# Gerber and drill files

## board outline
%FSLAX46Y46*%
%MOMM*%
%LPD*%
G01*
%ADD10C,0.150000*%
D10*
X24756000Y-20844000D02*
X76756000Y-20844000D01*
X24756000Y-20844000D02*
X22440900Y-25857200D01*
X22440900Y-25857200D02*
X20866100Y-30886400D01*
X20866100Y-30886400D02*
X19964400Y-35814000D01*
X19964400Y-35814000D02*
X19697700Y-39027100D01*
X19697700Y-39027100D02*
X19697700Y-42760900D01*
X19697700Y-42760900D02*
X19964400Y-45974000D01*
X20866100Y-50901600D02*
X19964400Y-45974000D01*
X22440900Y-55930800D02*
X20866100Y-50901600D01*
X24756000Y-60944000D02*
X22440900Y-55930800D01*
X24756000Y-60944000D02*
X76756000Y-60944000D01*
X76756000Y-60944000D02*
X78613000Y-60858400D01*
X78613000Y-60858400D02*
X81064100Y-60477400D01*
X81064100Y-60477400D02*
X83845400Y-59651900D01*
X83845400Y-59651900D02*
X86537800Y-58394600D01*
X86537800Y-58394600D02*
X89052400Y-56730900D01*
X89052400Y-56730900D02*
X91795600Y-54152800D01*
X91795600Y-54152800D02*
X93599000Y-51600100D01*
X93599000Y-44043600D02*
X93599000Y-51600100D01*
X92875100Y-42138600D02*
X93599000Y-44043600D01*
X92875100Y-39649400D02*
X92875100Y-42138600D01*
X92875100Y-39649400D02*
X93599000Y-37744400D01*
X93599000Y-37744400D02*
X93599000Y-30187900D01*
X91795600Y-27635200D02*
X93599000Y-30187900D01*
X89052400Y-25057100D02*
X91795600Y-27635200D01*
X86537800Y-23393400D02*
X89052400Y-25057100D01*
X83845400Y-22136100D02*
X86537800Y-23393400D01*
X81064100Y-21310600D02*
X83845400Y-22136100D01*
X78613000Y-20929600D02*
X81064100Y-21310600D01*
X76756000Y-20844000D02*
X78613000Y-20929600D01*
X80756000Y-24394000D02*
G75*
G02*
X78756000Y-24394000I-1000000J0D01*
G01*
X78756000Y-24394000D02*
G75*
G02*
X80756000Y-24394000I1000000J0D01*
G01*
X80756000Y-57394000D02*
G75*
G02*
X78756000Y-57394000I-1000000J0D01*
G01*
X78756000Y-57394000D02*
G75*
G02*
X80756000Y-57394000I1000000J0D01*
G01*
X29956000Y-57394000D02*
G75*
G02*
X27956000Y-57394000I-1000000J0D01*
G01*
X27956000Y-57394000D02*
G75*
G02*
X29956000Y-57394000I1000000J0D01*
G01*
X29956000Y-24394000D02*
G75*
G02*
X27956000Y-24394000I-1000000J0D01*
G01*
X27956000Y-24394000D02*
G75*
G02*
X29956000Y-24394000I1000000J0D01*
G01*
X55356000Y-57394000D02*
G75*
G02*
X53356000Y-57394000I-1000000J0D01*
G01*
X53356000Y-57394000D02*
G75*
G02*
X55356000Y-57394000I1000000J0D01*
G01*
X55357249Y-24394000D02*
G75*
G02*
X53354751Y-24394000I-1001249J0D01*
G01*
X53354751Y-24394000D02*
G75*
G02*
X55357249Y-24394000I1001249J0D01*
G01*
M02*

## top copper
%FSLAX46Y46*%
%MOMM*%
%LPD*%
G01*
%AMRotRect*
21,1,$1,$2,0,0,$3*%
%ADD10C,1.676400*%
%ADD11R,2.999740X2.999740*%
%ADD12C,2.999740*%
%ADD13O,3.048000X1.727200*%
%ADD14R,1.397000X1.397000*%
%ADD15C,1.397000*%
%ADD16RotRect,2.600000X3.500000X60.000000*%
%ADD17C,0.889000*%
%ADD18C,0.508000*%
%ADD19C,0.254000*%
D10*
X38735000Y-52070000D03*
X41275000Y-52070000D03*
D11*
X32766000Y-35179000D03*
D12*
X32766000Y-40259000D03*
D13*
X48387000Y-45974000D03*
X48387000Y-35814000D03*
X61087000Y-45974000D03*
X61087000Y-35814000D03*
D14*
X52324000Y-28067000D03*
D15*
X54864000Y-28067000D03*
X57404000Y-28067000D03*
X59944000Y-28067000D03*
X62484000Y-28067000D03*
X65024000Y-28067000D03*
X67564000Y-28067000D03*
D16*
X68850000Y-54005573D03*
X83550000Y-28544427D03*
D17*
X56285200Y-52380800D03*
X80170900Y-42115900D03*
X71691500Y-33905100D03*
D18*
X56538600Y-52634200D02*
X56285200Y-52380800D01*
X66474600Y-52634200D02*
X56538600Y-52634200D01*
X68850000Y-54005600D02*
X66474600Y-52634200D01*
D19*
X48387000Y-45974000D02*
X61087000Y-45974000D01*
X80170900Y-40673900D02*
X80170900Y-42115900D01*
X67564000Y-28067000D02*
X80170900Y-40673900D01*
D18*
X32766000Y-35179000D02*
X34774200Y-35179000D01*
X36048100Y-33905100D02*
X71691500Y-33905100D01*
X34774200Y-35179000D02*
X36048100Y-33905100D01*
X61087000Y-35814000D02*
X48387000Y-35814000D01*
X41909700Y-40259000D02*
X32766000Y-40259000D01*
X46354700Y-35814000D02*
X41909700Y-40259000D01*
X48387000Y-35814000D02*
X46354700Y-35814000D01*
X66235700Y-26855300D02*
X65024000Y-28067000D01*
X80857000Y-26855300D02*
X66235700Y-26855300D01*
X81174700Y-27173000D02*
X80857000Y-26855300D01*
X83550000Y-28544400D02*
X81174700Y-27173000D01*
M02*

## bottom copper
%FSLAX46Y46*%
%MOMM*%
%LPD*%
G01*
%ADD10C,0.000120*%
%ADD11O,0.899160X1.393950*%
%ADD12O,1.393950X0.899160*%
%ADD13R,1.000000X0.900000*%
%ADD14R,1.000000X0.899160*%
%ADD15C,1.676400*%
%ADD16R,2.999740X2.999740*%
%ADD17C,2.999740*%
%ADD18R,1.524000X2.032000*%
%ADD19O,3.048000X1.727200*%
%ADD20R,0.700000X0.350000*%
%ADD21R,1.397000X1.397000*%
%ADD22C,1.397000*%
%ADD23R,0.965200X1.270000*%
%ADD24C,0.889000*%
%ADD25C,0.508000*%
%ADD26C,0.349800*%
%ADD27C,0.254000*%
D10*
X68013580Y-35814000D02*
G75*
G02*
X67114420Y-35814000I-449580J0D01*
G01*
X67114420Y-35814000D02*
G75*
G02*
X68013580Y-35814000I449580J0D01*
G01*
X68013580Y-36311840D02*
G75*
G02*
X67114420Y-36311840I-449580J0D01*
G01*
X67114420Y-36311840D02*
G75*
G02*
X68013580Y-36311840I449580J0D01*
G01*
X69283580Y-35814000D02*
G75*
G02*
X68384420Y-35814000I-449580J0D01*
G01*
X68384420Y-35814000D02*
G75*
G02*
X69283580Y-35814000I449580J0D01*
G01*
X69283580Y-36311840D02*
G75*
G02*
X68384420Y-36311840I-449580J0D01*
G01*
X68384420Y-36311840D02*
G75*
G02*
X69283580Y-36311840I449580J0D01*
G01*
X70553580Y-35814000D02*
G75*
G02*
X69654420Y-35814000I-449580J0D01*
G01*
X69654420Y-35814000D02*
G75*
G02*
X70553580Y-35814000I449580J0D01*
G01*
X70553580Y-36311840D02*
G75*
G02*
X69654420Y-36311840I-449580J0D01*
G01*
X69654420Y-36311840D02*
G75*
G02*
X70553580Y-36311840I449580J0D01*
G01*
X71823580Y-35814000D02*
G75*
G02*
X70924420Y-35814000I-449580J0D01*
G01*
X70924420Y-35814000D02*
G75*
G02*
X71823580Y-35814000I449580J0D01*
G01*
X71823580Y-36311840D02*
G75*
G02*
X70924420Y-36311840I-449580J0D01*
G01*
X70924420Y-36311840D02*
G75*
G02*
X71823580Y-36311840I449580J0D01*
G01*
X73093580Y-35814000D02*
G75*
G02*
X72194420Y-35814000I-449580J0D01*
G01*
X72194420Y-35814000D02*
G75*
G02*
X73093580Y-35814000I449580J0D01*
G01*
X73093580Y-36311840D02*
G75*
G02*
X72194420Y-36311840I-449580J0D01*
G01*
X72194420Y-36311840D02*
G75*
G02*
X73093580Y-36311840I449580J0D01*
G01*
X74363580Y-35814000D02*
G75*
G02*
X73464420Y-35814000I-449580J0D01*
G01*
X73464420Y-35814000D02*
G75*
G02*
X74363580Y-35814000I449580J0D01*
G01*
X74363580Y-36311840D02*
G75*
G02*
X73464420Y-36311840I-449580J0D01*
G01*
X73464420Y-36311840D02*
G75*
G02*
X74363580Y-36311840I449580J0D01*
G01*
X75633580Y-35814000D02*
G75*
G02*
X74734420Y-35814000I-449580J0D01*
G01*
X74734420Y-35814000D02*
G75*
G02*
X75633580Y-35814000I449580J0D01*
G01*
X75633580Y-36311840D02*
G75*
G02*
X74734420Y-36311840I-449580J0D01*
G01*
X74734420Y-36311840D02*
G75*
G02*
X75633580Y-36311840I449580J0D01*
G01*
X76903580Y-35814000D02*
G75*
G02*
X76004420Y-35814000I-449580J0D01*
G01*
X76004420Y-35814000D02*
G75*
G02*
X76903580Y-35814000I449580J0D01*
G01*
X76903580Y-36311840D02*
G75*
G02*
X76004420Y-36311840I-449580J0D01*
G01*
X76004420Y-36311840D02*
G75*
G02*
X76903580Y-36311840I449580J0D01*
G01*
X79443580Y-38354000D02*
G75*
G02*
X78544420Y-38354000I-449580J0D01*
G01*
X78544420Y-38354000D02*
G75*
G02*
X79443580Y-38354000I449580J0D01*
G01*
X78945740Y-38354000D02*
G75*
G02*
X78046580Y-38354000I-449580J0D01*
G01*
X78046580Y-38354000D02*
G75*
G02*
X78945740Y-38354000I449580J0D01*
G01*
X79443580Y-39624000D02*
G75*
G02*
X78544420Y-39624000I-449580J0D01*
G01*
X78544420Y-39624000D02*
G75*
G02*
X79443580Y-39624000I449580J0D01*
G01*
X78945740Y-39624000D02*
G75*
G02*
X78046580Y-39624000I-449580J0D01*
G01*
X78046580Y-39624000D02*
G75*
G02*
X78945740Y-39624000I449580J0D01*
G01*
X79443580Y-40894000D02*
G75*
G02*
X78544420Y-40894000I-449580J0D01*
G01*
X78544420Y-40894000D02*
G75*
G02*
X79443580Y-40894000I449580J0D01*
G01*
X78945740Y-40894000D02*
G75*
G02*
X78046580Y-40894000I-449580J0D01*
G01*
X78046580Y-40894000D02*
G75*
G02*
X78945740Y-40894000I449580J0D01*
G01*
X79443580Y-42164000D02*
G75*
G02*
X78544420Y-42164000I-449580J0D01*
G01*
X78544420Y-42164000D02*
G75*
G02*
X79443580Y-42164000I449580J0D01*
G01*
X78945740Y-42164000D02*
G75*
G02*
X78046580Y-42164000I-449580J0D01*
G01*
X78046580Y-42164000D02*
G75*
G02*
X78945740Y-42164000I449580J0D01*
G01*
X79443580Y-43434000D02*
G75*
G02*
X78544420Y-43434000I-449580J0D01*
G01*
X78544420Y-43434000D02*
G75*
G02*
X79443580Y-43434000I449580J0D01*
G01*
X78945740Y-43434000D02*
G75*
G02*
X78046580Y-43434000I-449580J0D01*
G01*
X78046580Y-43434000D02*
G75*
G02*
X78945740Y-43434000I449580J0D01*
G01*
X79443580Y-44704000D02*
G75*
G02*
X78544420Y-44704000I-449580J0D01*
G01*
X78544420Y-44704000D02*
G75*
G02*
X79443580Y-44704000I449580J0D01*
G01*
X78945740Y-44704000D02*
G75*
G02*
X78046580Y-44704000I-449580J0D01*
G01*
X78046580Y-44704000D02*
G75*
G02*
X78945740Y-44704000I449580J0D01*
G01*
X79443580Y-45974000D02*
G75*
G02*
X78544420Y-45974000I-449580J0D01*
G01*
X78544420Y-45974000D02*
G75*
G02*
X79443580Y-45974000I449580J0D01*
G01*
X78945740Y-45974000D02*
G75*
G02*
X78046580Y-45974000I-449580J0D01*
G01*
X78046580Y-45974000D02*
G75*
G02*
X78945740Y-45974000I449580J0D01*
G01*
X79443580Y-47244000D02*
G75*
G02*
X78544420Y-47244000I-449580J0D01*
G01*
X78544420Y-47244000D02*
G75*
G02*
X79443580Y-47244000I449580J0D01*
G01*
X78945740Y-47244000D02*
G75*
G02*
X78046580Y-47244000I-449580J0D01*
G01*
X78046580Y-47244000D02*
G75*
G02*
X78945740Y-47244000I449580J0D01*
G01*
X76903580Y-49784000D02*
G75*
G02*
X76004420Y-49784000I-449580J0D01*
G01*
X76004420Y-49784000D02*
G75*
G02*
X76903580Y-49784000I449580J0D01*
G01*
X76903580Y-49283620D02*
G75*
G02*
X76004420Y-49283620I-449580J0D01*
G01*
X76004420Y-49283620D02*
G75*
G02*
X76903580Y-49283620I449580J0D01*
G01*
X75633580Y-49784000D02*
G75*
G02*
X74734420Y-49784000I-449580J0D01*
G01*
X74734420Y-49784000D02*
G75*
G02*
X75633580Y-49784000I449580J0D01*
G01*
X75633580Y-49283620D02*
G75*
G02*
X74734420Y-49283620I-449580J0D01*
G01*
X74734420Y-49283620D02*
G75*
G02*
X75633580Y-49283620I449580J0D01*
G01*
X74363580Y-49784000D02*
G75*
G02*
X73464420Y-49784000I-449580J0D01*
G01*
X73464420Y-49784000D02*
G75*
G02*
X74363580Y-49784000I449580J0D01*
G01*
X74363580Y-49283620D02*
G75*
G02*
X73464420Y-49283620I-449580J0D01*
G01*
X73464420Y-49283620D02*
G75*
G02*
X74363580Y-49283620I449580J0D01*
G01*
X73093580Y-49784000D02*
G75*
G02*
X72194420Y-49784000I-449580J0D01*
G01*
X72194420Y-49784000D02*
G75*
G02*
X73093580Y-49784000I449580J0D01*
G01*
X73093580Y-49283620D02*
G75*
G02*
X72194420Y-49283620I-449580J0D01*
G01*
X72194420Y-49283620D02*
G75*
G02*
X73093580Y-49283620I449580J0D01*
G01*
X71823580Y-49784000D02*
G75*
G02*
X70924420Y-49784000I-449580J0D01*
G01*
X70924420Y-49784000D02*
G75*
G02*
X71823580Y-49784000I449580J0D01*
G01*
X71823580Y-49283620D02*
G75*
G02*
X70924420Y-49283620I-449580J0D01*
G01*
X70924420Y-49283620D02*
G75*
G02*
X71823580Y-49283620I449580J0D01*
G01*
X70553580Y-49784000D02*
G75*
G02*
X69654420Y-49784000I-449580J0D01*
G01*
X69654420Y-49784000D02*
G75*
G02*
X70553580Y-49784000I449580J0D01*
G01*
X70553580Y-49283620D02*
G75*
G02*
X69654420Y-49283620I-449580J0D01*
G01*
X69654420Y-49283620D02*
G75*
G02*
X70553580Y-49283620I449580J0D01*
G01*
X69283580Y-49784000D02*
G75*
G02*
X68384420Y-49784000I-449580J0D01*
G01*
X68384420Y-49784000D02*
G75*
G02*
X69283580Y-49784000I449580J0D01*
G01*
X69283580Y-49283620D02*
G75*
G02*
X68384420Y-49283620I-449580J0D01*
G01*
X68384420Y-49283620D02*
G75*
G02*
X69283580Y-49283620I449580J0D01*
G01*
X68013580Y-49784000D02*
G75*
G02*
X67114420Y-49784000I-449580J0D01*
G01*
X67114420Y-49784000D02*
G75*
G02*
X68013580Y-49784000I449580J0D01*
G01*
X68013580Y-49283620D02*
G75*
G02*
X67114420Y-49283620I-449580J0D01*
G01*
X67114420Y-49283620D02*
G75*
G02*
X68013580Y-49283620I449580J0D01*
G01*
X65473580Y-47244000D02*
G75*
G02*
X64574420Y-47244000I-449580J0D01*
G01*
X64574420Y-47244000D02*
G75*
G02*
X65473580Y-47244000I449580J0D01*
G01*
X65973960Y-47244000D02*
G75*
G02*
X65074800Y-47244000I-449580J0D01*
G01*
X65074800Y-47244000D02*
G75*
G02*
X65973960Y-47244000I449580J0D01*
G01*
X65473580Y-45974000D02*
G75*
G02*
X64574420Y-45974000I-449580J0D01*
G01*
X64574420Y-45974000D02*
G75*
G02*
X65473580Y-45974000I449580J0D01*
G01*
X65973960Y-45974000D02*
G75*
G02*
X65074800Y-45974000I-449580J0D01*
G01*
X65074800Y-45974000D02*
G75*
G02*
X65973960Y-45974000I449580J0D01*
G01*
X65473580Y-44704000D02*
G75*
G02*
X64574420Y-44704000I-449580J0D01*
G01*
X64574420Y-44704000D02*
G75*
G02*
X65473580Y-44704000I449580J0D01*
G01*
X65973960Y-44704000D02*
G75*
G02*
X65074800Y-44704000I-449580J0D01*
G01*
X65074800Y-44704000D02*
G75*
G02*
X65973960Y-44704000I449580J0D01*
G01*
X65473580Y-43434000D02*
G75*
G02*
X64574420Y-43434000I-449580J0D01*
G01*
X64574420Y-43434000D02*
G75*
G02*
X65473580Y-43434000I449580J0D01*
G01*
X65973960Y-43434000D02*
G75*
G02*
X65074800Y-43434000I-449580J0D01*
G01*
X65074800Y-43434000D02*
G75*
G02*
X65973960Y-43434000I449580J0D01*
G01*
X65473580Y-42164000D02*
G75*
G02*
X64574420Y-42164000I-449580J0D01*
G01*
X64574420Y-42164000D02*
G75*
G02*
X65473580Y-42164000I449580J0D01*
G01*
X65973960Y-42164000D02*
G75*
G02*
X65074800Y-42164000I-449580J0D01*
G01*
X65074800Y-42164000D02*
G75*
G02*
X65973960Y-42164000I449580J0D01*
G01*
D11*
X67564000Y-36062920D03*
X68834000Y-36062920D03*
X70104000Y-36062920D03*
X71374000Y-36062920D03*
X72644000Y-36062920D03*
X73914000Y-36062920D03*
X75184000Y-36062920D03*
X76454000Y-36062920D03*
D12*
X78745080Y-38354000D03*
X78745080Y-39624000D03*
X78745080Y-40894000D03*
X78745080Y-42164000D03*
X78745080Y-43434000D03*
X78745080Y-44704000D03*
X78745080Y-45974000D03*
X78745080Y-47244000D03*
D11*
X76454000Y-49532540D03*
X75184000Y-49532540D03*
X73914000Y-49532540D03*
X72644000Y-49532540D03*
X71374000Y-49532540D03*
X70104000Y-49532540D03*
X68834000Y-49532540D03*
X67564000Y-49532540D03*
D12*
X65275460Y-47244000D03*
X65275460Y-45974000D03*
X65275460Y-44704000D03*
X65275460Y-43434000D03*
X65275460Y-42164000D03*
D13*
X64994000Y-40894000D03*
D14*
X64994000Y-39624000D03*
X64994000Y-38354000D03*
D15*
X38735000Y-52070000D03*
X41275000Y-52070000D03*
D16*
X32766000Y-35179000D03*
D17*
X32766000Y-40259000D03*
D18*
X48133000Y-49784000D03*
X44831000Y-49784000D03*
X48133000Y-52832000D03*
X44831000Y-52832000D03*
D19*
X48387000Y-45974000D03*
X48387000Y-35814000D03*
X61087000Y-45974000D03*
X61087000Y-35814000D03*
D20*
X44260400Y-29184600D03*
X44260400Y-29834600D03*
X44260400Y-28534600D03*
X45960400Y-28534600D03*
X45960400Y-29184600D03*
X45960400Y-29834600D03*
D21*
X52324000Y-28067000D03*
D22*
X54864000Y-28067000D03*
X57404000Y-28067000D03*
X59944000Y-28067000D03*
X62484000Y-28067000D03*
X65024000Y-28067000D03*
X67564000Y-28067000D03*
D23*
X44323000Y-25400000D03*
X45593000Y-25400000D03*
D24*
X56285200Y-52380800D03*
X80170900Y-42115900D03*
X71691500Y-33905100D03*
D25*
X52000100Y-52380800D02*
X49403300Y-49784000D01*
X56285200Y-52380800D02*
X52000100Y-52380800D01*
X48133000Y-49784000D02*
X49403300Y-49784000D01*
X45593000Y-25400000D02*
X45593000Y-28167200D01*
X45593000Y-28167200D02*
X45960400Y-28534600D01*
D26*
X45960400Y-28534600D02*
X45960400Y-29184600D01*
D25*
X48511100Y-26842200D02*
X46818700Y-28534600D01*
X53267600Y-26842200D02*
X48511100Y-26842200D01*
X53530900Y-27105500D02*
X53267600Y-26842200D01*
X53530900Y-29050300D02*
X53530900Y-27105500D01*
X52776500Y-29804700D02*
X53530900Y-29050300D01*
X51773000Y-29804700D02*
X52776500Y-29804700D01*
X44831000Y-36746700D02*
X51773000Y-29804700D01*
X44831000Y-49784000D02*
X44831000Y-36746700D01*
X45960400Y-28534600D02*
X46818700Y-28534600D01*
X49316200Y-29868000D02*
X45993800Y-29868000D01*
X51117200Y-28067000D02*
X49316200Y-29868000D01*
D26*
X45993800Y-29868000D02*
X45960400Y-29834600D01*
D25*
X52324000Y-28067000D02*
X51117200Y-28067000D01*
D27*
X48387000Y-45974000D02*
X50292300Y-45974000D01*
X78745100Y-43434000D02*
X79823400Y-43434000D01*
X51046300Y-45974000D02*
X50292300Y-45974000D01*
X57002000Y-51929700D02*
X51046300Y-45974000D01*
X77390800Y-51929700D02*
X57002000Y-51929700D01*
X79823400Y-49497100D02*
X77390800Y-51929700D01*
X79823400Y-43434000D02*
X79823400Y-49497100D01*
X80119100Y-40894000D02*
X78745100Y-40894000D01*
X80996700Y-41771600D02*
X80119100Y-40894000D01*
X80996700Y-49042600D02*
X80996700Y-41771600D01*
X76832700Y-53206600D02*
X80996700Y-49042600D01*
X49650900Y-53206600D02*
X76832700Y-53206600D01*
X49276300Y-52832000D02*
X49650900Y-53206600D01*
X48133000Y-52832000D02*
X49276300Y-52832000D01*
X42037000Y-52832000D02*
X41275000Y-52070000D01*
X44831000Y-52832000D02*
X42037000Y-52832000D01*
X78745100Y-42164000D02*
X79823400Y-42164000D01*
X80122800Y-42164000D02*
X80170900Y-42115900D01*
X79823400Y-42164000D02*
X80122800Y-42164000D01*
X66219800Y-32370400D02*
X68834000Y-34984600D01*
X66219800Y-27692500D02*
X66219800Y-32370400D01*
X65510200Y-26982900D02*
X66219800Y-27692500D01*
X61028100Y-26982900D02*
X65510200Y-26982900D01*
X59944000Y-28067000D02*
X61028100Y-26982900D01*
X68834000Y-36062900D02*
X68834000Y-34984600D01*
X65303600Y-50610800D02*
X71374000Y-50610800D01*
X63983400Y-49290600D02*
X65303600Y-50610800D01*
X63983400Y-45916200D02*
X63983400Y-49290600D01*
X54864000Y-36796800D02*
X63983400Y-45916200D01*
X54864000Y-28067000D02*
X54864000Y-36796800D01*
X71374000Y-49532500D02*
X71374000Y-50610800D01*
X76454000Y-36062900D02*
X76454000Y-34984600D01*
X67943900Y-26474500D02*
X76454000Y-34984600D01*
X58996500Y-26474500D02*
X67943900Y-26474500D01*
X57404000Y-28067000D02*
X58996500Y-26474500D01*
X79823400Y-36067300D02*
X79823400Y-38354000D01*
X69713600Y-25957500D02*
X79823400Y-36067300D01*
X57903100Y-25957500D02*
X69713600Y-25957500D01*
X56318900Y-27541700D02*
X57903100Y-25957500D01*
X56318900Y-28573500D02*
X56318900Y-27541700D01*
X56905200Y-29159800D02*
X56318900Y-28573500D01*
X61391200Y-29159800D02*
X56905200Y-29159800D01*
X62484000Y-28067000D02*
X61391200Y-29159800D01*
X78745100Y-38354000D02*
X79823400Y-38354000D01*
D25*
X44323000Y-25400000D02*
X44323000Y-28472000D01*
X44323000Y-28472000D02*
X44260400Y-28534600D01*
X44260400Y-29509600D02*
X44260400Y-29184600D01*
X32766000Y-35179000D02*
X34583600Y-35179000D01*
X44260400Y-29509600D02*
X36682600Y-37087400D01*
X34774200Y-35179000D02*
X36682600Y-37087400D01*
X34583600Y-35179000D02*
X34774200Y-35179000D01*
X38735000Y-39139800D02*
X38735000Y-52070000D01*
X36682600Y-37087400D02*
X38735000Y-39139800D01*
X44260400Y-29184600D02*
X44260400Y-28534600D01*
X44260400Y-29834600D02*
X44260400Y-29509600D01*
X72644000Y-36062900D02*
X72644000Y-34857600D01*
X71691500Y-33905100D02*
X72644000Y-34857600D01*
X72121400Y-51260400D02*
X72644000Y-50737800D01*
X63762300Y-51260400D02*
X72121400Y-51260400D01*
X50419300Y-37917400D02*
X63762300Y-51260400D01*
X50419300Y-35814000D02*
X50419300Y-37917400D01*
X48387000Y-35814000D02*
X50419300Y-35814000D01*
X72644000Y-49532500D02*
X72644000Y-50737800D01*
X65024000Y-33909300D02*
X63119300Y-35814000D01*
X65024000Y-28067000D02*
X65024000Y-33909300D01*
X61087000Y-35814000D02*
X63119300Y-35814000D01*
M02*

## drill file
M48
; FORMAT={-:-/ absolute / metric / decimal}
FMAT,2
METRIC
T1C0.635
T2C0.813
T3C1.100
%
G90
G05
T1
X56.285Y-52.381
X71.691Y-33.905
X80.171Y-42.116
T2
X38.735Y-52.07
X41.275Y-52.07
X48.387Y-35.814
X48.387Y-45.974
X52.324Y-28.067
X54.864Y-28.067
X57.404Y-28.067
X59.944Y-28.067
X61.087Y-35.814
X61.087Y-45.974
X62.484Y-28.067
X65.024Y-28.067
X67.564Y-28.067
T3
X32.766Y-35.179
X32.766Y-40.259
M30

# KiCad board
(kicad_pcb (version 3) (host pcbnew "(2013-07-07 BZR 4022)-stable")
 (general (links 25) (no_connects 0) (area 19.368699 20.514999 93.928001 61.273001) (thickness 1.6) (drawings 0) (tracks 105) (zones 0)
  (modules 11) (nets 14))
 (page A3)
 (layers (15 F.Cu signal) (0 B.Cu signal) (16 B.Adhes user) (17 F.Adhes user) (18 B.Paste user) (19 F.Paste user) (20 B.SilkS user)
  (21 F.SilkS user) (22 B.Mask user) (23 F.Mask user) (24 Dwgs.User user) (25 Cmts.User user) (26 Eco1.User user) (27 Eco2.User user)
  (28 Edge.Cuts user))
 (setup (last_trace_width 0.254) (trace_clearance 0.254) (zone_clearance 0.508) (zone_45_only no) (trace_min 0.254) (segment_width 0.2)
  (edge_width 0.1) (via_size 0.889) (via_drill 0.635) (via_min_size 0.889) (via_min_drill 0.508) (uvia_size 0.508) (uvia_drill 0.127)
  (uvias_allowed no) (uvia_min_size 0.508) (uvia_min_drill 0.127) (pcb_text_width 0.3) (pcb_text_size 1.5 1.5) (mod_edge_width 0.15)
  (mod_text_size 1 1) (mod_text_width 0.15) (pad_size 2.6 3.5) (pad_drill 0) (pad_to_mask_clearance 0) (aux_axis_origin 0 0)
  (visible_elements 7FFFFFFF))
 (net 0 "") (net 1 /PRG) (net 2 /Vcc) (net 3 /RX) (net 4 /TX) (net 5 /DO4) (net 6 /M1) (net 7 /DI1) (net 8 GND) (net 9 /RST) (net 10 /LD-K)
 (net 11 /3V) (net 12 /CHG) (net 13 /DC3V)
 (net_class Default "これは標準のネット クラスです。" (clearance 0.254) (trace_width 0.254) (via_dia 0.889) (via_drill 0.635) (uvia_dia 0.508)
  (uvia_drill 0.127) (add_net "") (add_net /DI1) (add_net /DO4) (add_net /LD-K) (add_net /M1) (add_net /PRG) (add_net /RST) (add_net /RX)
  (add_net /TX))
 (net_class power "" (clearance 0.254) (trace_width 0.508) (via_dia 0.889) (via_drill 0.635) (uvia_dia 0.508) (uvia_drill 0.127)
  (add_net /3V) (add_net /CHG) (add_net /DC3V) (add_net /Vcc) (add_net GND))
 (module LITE (layer B.Cu) (at 78.994 35.814 270)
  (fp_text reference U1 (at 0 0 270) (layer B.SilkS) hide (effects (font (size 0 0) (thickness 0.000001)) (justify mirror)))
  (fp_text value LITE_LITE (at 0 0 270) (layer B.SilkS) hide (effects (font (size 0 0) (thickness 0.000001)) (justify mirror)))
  (fp_circle (center 0 11.43) (end 0.44958 11.43) (layer B.Cu) (width 0.00012))
  (fp_circle (center 0.49784 11.43) (end 0.94742 11.43) (layer B.Cu) (width 0.00012))
  (fp_circle (center 0 10.16) (end 0.44958 10.16) (layer B.Cu) (width 0.00012))
  (fp_circle (center 0.49784 10.16) (end 0.94742 10.16) (layer B.Cu) (width 0.00012))
  (fp_circle (center 0 8.89) (end 0.44958 8.89) (layer B.Cu) (width 0.00012))
  (fp_circle (center 0.49784 8.89) (end 0.94742 8.89) (layer B.Cu) (width 0.00012))
  (fp_circle (center 0 7.62) (end 0.44958 7.62) (layer B.Cu) (width 0.00012))
  (fp_circle (center 0.49784 7.62) (end 0.94742 7.62) (layer B.Cu) (width 0.00012))
  (fp_circle (center 0 6.35) (end 0.44958 6.35) (layer B.Cu) (width 0.00012))
  (fp_circle (center 0.49784 6.35) (end 0.94742 6.35) (layer B.Cu) (width 0.00012))
  (fp_circle (center 0 5.08) (end 0.44958 5.08) (layer B.Cu) (width 0.00012))
  (fp_circle (center 0.49784 5.08) (end 0.94742 5.08) (layer B.Cu) (width 0.00012))
  (fp_circle (center 0 3.81) (end 0.44958 3.81) (layer B.Cu) (width 0.00012))
  (fp_circle (center 0.49784 3.81) (end 0.94742 3.81) (layer B.Cu) (width 0.00012))
  (fp_circle (center 0 2.54) (end 0.44958 2.54) (layer B.Cu) (width 0.00012))
  (fp_circle (center 0.49784 2.54) (end 0.94742 2.54) (layer B.Cu) (width 0.00012))
  (fp_circle (center 2.54 0) (end 2.98958 0) (layer B.Cu) (width 0.00012))
  (fp_circle (center 2.54 0.49784) (end 2.98958 0.49784) (layer B.Cu) (width 0.00012))
  (fp_circle (center 3.81 0) (end 4.25958 0) (layer B.Cu) (width 0.00012))
  (fp_circle (center 3.81 0.49784) (end 4.25958 0.49784) (layer B.Cu) (width 0.00012))
  (fp_circle (center 5.08 0) (end 5.52958 0) (layer B.Cu) (width 0.00012))
  (fp_circle (center 5.08 0.49784) (end 5.52958 0.49784) (layer B.Cu) (width 0.00012))
  (fp_circle (center 6.35 0) (end 6.79958 0) (layer B.Cu) (width 0.00012))
  (fp_circle (center 6.35 0.49784) (end 6.79958 0.49784) (layer B.Cu) (width 0.00012))
  (fp_circle (center 7.62 0) (end 8.06958 0) (layer B.Cu) (width 0.00012))
  (fp_circle (center 7.62 0.49784) (end 8.06958 0.49784) (layer B.Cu) (width 0.00012))
  (fp_circle (center 8.89 0) (end 9.33958 0) (layer B.Cu) (width 0.00012))
  (fp_circle (center 8.89 0.49784) (end 9.33958 0.49784) (layer B.Cu) (width 0.00012))
  (fp_circle (center 10.16 0) (end 10.60958 0) (layer B.Cu) (width 0.00012))
  (fp_circle (center 10.16 0.49784) (end 10.60958 0.49784) (layer B.Cu) (width 0.00012))
  (fp_circle (center 11.43 0) (end 11.87958 0) (layer B.Cu) (width 0.00012))
  (fp_circle (center 11.43 0.49784) (end 11.87958 0.49784) (layer B.Cu) (width 0.00012))
  (fp_circle (center 13.97 2.54) (end 14.41958 2.54) (layer B.Cu) (width 0.00012))
  (fp_circle (center 13.46962 2.54) (end 13.9192 2.54) (layer B.Cu) (width 0.00012))
  (fp_circle (center 13.97 3.81) (end 14.41958 3.81) (layer B.Cu) (width 0.00012))
  (fp_circle (center 13.46962 3.81) (end 13.9192 3.81) (layer B.Cu) (width 0.00012))
  (fp_circle (center 13.97 5.08) (end 14.41958 5.08) (layer B.Cu) (width 0.00012))
  (fp_circle (center 13.46962 5.08) (end 13.9192 5.08) (layer B.Cu) (width 0.00012))
  (fp_circle (center 13.97 6.35) (end 14.41958 6.35) (layer B.Cu) (width 0.00012))
  (fp_circle (center 13.46962 6.35) (end 13.9192 6.35) (layer B.Cu) (width 0.00012))
  (fp_circle (center 13.97 7.62) (end 14.41958 7.62) (layer B.Cu) (width 0.00012))
  (fp_circle (center 13.46962 7.62) (end 13.9192 7.62) (layer B.Cu) (width 0.00012))
  (fp_circle (center 13.97 8.89) (end 14.41958 8.89) (layer B.Cu) (width 0.00012))
  (fp_circle (center 13.46962 8.89) (end 13.9192 8.89) (layer B.Cu) (width 0.00012))
  (fp_circle (center 13.97 10.16) (end 14.41958 10.16) (layer B.Cu) (width 0.00012))
  (fp_circle (center 13.46962 10.16) (end 13.9192 10.16) (layer B.Cu) (width 0.00012))
  (fp_circle (center 13.97 11.43) (end 14.41958 11.43) (layer B.Cu) (width 0.00012))
  (fp_circle (center 13.46962 11.43) (end 13.9192 11.43) (layer B.Cu) (width 0.00012))
  (fp_circle (center 11.43 13.97) (end 11.87958 13.97) (layer B.Cu) (width 0.00012))
  (fp_circle (center 11.43 13.46962) (end 11.87958 13.46962) (layer B.Cu) (width 0.00012))
  (fp_circle (center 10.16 13.97) (end 10.60958 13.97) (layer B.Cu) (width 0.00012))
  (fp_circle (center 10.16 13.46962) (end 10.60958 13.46962) (layer B.Cu) (width 0.00012))
  (fp_circle (center 8.89 13.97) (end 9.33958 13.97) (layer B.Cu) (width 0.00012))
  (fp_circle (center 8.89 13.46962) (end 9.33958 13.46962) (layer B.Cu) (width 0.00012))
  (fp_circle (center 7.62 13.97) (end 8.06958 13.97) (layer B.Cu) (width 0.00012))
  (fp_circle (center 7.62 13.46962) (end 8.06958 13.46962) (layer B.Cu) (width 0.00012))
  (fp_circle (center 6.35 13.97) (end 6.79958 13.97) (layer B.Cu) (width 0.00012))
  (fp_circle (center 6.35 13.46962) (end 6.79958 13.46962) (layer B.Cu) (width 0.00012))
  (pad 1 smd oval (at 0.24892 11.43 270) (size 1.39395 0.89916) (layers B.Cu B.Paste B.Mask))
  (pad 2 smd oval (at 0.24892 10.16 270) (size 1.39395 0.89916) (layers B.Cu B.Paste B.Mask) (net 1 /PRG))
  (pad 3 smd oval (at 0.24892 8.89 270) (size 1.39395 0.89916) (layers B.Cu B.Paste B.Mask))
  (pad 4 smd oval (at 0.24892 7.62 270) (size 1.39395 0.89916) (layers B.Cu B.Paste B.Mask))
  (pad 5 smd oval (at 0.24892 6.35 270) (size 1.39395 0.89916) (layers B.Cu B.Paste B.Mask) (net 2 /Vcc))
  (pad 6 smd oval (at 0.24892 5.08 270) (size 1.39395 0.89916) (layers B.Cu B.Paste B.Mask))
  (pad 7 smd oval (at 0.24892 3.81 270) (size 1.39395 0.89916) (layers B.Cu B.Paste B.Mask))
  (pad 8 smd oval (at 0.24892 2.54 270) (size 1.39395 0.89916) (layers B.Cu B.Paste B.Mask) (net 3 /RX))
  (pad 9 smd oval (at 2.54 0.24892 180) (size 1.39395 0.89916) (layers B.Cu B.Paste B.Mask) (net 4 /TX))
  (pad 10 smd oval (at 3.81 0.24892 180) (size 1.39395 0.89916) (layers B.Cu B.Paste B.Mask))
  (pad 11 smd oval (at 5.08 0.24892 180) (size 1.39395 0.89916) (layers B.Cu B.Paste B.Mask) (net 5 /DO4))
  (pad 12 smd oval (at 6.35 0.24892 180) (size 1.39395 0.89916) (layers B.Cu B.Paste B.Mask) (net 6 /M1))
  (pad 13 smd oval (at 7.62 0.24892 180) (size 1.39395 0.89916) (layers B.Cu B.Paste B.Mask) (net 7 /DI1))
  (pad 14 smd oval (at 8.89 0.24892 180) (size 1.39395 0.89916) (layers B.Cu B.Paste B.Mask))
  (pad 15 smd oval (at 10.16 0.24892 180) (size 1.39395 0.89916) (layers B.Cu B.Paste B.Mask))
  (pad 16 smd oval (at 11.43 0.24892 180) (size 1.39395 0.89916) (layers B.Cu B.Paste B.Mask))
  (pad 17 smd oval (at 13.71854 2.54 90) (size 1.39395 0.89916) (layers B.Cu B.Paste B.Mask))
  (pad 18 smd oval (at 13.71854 3.81 90) (size 1.39395 0.89916) (layers B.Cu B.Paste B.Mask))
  (pad 19 smd oval (at 13.71854 5.08 90) (size 1.39395 0.89916) (layers B.Cu B.Paste B.Mask))
  (pad 20 smd oval (at 13.71854 6.35 90) (size 1.39395 0.89916) (layers B.Cu B.Paste B.Mask) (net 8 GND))
  (pad 21 smd oval (at 13.71854 7.62 90) (size 1.39395 0.89916) (layers B.Cu B.Paste B.Mask) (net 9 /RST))
  (pad 22 smd oval (at 13.71854 8.89 90) (size 1.39395 0.89916) (layers B.Cu B.Paste B.Mask))
  (pad 23 smd oval (at 13.71854 10.16 90) (size 1.39395 0.89916) (layers B.Cu B.Paste B.Mask))
  (pad 24 smd oval (at 13.71854 11.43 90) (size 1.39395 0.89916) (layers B.Cu B.Paste B.Mask))
  (pad 25 smd oval (at 11.43 13.71854) (size 1.39395 0.89916) (layers B.Cu B.Paste B.Mask))
  (pad 26 smd oval (at 10.16 13.71854) (size 1.39395 0.89916) (layers B.Cu B.Paste B.Mask))
  (pad 27 smd oval (at 8.89 13.71854) (size 1.39395 0.89916) (layers B.Cu B.Paste B.Mask))
  (pad 28 smd oval (at 7.62 13.71854) (size 1.39395 0.89916) (layers B.Cu B.Paste B.Mask))
  (pad 29 smd oval (at 6.35 13.71854) (size 1.39395 0.89916) (layers B.Cu B.Paste B.Mask))
  (pad 30 smd rect (at 5.08 14) (size 1 0.9) (layers B.Cu B.Paste B.Mask))
  (pad 31 smd rect (at 3.81 14) (size 1 0.89916) (layers B.Cu B.Paste B.Mask))
  (pad 32 smd rect (at 2.54 14) (size 1 0.89916) (layers B.Cu B.Paste B.Mask)))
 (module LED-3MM (layer F.Cu) (at 40.005 52.07)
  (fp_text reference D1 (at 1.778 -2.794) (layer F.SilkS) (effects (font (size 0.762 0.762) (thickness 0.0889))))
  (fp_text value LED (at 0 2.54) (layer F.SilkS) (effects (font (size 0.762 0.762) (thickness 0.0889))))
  (pad 1 thru_hole circle (at -1.27 0) (size 1.6764 1.6764) (drill 0.8128) (layers *.Cu *.Mask F.SilkS) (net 2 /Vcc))
  (pad 2 thru_hole circle (at 1.27 0) (size 1.6764 1.6764) (drill 0.8128) (layers *.Cu *.Mask F.SilkS) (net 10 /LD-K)))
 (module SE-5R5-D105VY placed (layer F.Cu) (at 32.766 37.719 180)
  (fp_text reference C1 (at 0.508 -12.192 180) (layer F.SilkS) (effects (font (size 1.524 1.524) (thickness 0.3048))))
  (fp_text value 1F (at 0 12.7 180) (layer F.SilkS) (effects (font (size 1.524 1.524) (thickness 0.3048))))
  (pad 1 thru_hole rect (at 0 2.54 180) (size 2.99974 2.99974) (drill 1.1) (layers *.Cu *.Mask F.SilkS) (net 2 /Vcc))
  (pad 2 thru_hole circle (at 0 -2.54 180) (size 2.99974 2.99974) (drill 1.1) (layers *.Cu *.Mask F.SilkS) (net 8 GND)))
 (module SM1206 (layer B.Cu) (at 46.482 49.784 180)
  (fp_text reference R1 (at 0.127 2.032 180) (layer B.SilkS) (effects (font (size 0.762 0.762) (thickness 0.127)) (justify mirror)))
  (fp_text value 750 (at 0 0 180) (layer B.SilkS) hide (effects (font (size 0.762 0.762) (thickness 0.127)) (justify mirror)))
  (pad 1 smd rect (at -1.651 0 180) (size 1.524 2.032) (layers B.Cu B.Paste B.Mask) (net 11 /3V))
  (pad 2 smd rect (at 1.651 0 180) (size 1.524 2.032) (layers B.Cu B.Paste B.Mask) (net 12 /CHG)))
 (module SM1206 (layer B.Cu) (at 46.482 52.832 180)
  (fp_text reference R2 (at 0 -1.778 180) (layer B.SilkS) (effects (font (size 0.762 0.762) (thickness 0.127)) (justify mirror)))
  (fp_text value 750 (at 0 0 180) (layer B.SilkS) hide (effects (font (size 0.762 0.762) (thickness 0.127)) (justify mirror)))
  (pad 1 smd rect (at -1.651 0 180) (size 1.524 2.032) (layers B.Cu B.Paste B.Mask) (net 5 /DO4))
  (pad 2 smd rect (at 1.651 0 180) (size 1.524 2.032) (layers B.Cu B.Paste B.Mask) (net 10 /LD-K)))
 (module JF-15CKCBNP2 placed (layer F.Cu) (at 54.737 40.894 180)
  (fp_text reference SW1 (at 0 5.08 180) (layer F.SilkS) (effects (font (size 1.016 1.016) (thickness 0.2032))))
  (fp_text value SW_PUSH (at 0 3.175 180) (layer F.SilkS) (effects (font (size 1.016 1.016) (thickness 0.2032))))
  (pad 1 thru_hole oval (at 6.35 -5.08 180) (size 3.048 1.7272) (drill 0.8128) (layers *.Cu *.Mask F.SilkS) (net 7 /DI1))
  (pad 2 thru_hole oval (at 6.35 5.08 180) (size 3.048 1.7272) (drill 0.8128) (layers *.Cu *.Mask F.SilkS) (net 8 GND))
  (pad 1 thru_hole oval (at -6.35 -5.08 180) (size 3.048 1.7272) (drill 0.8128) (layers *.Cu *.Mask F.SilkS) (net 7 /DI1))
  (pad 2 thru_hole oval (at -6.35 5.08 180) (size 3.048 1.7272) (drill 0.8128) (layers *.Cu *.Mask F.SilkS) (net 8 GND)))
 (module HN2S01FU (layer B.Cu) (at 45.1104 29.1846)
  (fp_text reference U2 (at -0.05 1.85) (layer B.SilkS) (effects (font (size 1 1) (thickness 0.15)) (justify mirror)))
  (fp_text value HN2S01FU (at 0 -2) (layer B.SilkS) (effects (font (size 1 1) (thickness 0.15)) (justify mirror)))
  (pad 2 smd rect (at -0.85 0) (size 0.7 0.35) (layers B.Cu B.Paste B.Mask) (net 2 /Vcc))
  (pad 1 smd rect (at -0.85 0.65) (size 0.7 0.35) (layers B.Cu B.Paste B.Mask) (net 2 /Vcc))
  (pad 3 smd rect (at -0.85 -0.65) (size 0.7 0.35) (layers B.Cu B.Paste B.Mask) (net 2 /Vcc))
  (pad 4 smd rect (at 0.85 -0.65) (size 0.7 0.35) (layers B.Cu B.Paste B.Mask) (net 12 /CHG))
  (pad 5 smd rect (at 0.85 0) (size 0.7 0.35) (layers B.Cu B.Paste B.Mask) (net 12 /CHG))
  (pad 6 smd rect (at 0.85 0.65) (size 0.7 0.35) (layers B.Cu B.Paste B.Mask) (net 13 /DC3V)))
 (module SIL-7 (layer F.Cu) (at 59.944 28.067)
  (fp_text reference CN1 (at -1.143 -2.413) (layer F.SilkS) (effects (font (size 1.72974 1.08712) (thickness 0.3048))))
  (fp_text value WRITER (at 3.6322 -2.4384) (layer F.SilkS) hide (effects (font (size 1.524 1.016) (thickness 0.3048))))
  (pad 1 thru_hole rect (at -7.62 0) (size 1.397 1.397) (drill 0.8128) (layers *.Cu *.Mask F.SilkS) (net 13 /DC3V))
  (pad 2 thru_hole circle (at -5.08 0) (size 1.397 1.397) (drill 0.8128) (layers *.Cu *.SilkS *.Mask) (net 9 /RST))
  (pad 3 thru_hole circle (at -2.54 0) (size 1.397 1.397) (drill 0.8128) (layers *.Cu *.SilkS *.Mask) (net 3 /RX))
  (pad 4 thru_hole circle (at 0 0) (size 1.397 1.397) (drill 0.8128) (layers *.Cu *.SilkS *.Mask) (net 1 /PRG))
  (pad 5 thru_hole circle (at 2.54 0) (size 1.397 1.397) (drill 0.8128) (layers *.Cu *.SilkS *.Mask) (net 4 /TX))
  (pad 6 thru_hole circle (at 5.08 0) (size 1.397 1.397) (drill 0.8128) (layers *.Cu *.SilkS *.Mask) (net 8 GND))
  (pad 7 thru_hole circle (at 7.62 0) (size 1.397 1.397) (drill 0.8128) (layers *.Cu *.SilkS *.Mask) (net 6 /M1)))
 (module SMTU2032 (layer F.Cu) (at 76.2 41.275 60)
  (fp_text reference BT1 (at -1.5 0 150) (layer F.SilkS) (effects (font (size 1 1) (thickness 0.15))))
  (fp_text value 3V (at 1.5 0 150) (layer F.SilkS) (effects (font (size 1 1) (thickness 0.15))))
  (pad 1 smd rect (at -14.7 0 60) (size 2.6 3.5) (layers F.Cu F.Paste F.Mask) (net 11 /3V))
  (pad 2 smd rect (at 14.7 0 60) (size 2.6 3.5) (layers F.Cu F.Paste F.Mask) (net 8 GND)))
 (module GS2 (layer B.Cu) (at 44.958 25.4 270)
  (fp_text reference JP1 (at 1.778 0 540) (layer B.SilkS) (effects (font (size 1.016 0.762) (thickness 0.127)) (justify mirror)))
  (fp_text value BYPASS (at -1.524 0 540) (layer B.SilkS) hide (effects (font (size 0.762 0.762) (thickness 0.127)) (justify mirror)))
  (pad 1 smd rect (at 0 0.635 270) (size 1.27 0.9652) (layers B.Cu B.Paste B.Mask) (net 2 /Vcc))
  (pad 2 smd rect (at 0 -0.635 270) (size 1.27 0.9652) (layers B.Cu B.Paste B.Mask) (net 12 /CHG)))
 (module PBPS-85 (layer F.Cu) (at 54.356 40.894)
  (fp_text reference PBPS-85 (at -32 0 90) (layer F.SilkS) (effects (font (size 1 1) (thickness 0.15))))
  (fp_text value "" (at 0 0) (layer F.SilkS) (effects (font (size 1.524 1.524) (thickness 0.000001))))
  (fp_line (start -29.6 -20.05) (end 22.4 -20.05) (layer Edge.Cuts) (width 0.15))
  (fp_line (start -29.6 -20.05) (end -31.9151 -15.0368) (layer Edge.Cuts) (width 0.15))
  (fp_line (start -31.9151 -15.0368) (end -33.4899 -10.0076) (layer Edge.Cuts) (width 0.15))
  (fp_line (start -33.4899 -10.0076) (end -34.3916 -5.08) (layer Edge.Cuts) (width 0.15))
  (fp_line (start -34.3916 -5.08) (end -34.6583 -1.8669) (layer Edge.Cuts) (width 0.15))
  (fp_line (start -34.6583 -1.8669) (end -34.6583 1.8669) (layer Edge.Cuts) (width 0.15))
  (fp_line (start -34.6583 1.8669) (end -34.3916 5.08) (layer Edge.Cuts) (width 0.15))
  (fp_line (start -33.4899 10.0076) (end -34.3916 5.08) (layer Edge.Cuts) (width 0.15))
  (fp_line (start -31.9151 15.0368) (end -33.4899 10.0076) (layer Edge.Cuts) (width 0.15))
  (fp_line (start -29.6 20.05) (end -31.9151 15.0368) (layer Edge.Cuts) (width 0.15))
  (fp_line (start -29.6 20.05) (end 22.4 20.05) (layer Edge.Cuts) (width 0.15))
  (fp_line (start 22.4 20.05) (end 24.257 19.9644) (layer Edge.Cuts) (width 0.15))
  (fp_line (start 24.257 19.9644) (end 26.7081 19.5834) (layer Edge.Cuts) (width 0.15))
  (fp_line (start 26.7081 19.5834) (end 29.4894 18.7579) (layer Edge.Cuts) (width 0.15))
  (fp_line (start 29.4894 18.7579) (end 32.1818 17.5006) (layer Edge.Cuts) (width 0.15))
  (fp_line (start 32.1818 17.5006) (end 34.6964 15.8369) (layer Edge.Cuts) (width 0.15))
  (fp_line (start 34.6964 15.8369) (end 37.4396 13.2588) (layer Edge.Cuts) (width 0.15))
  (fp_line (start 37.4396 13.2588) (end 39.243 10.7061) (layer Edge.Cuts) (width 0.15))
  (fp_line (start 39.243 3.1496) (end 39.243 10.7061) (layer Edge.Cuts) (width 0.15))
  (fp_line (start 38.5191 1.2446) (end 39.243 3.1496) (layer Edge.Cuts) (width 0.15))
  (fp_line (start 38.5191 -1.2446) (end 38.5191 1.2446) (layer Edge.Cuts) (width 0.15))
  (fp_line (start 38.5191 -1.2446) (end 39.243 -3.1496) (layer Edge.Cuts) (width 0.15))
  (fp_line (start 39.243 -3.1496) (end 39.243 -10.7061) (layer Edge.Cuts) (width 0.15))
  (fp_line (start 37.4396 -13.2588) (end 39.243 -10.7061) (layer Edge.Cuts) (width 0.15))
  (fp_line (start 34.6964 -15.8369) (end 37.4396 -13.2588) (layer Edge.Cuts) (width 0.15))
  (fp_line (start 32.1818 -17.5006) (end 34.6964 -15.8369) (layer Edge.Cuts) (width 0.15))
  (fp_line (start 29.4894 -18.7579) (end 32.1818 -17.5006) (layer Edge.Cuts) (width 0.15))
  (fp_line (start 26.7081 -19.5834) (end 29.4894 -18.7579) (layer Edge.Cuts) (width 0.15))
  (fp_line (start 24.257 -19.9644) (end 26.7081 -19.5834) (layer Edge.Cuts) (width 0.15))
  (fp_line (start 22.4 -20.05) (end 24.257 -19.9644) (layer Edge.Cuts) (width 0.15))
  (fp_circle (center 25.4 -16.5) (end 25.4 -15.5) (layer Edge.Cuts) (width 0.15))
  (fp_circle (center 25.4 16.5) (end 25.4 15.5) (layer Edge.Cuts) (width 0.15))
  (fp_circle (center -25.4 16.5) (end -25.4 15.5) (layer Edge.Cuts) (width 0.15))
  (fp_circle (center -25.4 -16.5) (end -25.4 -15.5) (layer Edge.Cuts) (width 0.15))
  (fp_circle (center 0 16.5) (end 0 17.5) (layer Edge.Cuts) (width 0.15))
  (fp_circle (center 0 -16.5) (end 0.05 -17.5) (layer Edge.Cuts) (width 0.15)))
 (via (at 56.2852 52.3808) (size 0.889) (layers F.Cu B.Cu) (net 11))
 (segment (start 56.5386 52.6342) (end 56.2852 52.3808) (width 0.508) (layer F.Cu) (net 11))
 (segment (start 66.4746 52.6342) (end 56.5386 52.6342) (width 0.508) (layer F.Cu) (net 11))
 (segment (start 52.0001 52.3808) (end 49.4033 49.784) (width 0.508) (layer B.Cu) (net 11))
 (segment (start 56.2852 52.3808) (end 52.0001 52.3808) (width 0.508) (layer B.Cu) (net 11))
 (segment (start 68.85 54.0056) (end 66.4746 52.6342) (width 0.508) (layer F.Cu) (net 11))
 (segment (start 48.133 49.784) (end 49.4033 49.784) (width 0.508) (layer B.Cu) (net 11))
 (segment (start 45.593 25.4) (end 45.593 28.1672) (width 0.508) (layer B.Cu) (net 12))
 (segment (start 45.593 28.1672) (end 45.9604 28.5346) (width 0.508) (layer B.Cu) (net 12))
 (segment (start 45.9604 28.5346) (end 45.9604 29.1846) (width 0.3498) (layer B.Cu) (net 12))
 (segment (start 48.5111 26.8422) (end 46.8187 28.5346) (width 0.508) (layer B.Cu) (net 12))
 (segment (start 53.2676 26.8422) (end 48.5111 26.8422) (width 0.508) (layer B.Cu) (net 12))
 (segment (start 53.5309 27.1055) (end 53.2676 26.8422) (width 0.508) (layer B.Cu) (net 12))
 (segment (start 53.5309 29.0503) (end 53.5309 27.1055) (width 0.508) (layer B.Cu) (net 12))
 (segment (start 52.7765 29.8047) (end 53.5309 29.0503) (width 0.508) (layer B.Cu) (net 12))
 (segment (start 51.773 29.8047) (end 52.7765 29.8047) (width 0.508) (layer B.Cu) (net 12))
 (segment (start 44.831 36.7467) (end 51.773 29.8047) (width 0.508) (layer B.Cu) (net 12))
 (segment (start 44.831 49.784) (end 44.831 36.7467) (width 0.508) (layer B.Cu) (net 12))
 (segment (start 45.9604 28.5346) (end 46.8187 28.5346) (width 0.508) (layer B.Cu) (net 12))
 (segment (start 49.3162 29.868) (end 45.9938 29.868) (width 0.508) (layer B.Cu) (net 13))
 (segment (start 51.1172 28.067) (end 49.3162 29.868) (width 0.508) (layer B.Cu) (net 13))
 (segment (start 45.9938 29.868) (end 45.9604 29.8346) (width 0.3498) (layer B.Cu) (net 13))
 (segment (start 52.324 28.067) (end 51.1172 28.067) (width 0.508) (layer B.Cu) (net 13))
 (segment (start 48.387 45.974) (end 61.087 45.974) (width 0.254) (layer F.Cu) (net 7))
 (segment (start 48.387 45.974) (end 50.2923 45.974) (width 0.254) (layer B.Cu) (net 7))
 (segment (start 78.7451 43.434) (end 79.8234 43.434) (width 0.254) (layer B.Cu) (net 7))
 (segment (start 51.0463 45.974) (end 50.2923 45.974) (width 0.254) (layer B.Cu) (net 7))
 (segment (start 57.002 51.9297) (end 51.0463 45.974) (width 0.254) (layer B.Cu) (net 7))
 (segment (start 77.3908 51.9297) (end 57.002 51.9297) (width 0.254) (layer B.Cu) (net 7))
 (segment (start 79.8234 49.4971) (end 77.3908 51.9297) (width 0.254) (layer B.Cu) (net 7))
 (segment (start 79.8234 43.434) (end 79.8234 49.4971) (width 0.254) (layer B.Cu) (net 7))
 (segment (start 80.1191 40.894) (end 78.7451 40.894) (width 0.254) (layer B.Cu) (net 5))
 (segment (start 80.9967 41.7716) (end 80.1191 40.894) (width 0.254) (layer B.Cu) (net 5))
 (segment (start 80.9967 49.0426) (end 80.9967 41.7716) (width 0.254) (layer B.Cu) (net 5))
 (segment (start 76.8327 53.2066) (end 80.9967 49.0426) (width 0.254) (layer B.Cu) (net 5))
 (segment (start 49.6509 53.2066) (end 76.8327 53.2066) (width 0.254) (layer B.Cu) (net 5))
 (segment (start 49.2763 52.832) (end 49.6509 53.2066) (width 0.254) (layer B.Cu) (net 5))
 (segment (start 48.133 52.832) (end 49.2763 52.832) (width 0.254) (layer B.Cu) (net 5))
 (segment (start 42.037 52.832) (end 41.275 52.07) (width 0.254) (layer B.Cu) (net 10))
 (segment (start 44.831 52.832) (end 42.037 52.832) (width 0.254) (layer B.Cu) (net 10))
 (via (at 80.1709 42.1159) (size 0.889) (layers F.Cu B.Cu) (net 6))
 (segment (start 78.7451 42.164) (end 79.8234 42.164) (width 0.254) (layer B.Cu) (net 6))
 (segment (start 80.1228 42.164) (end 80.1709 42.1159) (width 0.254) (layer B.Cu) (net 6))
 (segment (start 79.8234 42.164) (end 80.1228 42.164) (width 0.254) (layer B.Cu) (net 6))
 (segment (start 80.1709 40.6739) (end 80.1709 42.1159) (width 0.254) (layer F.Cu) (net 6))
 (segment (start 67.564 28.067) (end 80.1709 40.6739) (width 0.254) (layer F.Cu) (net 6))
 (segment (start 66.2198 32.3704) (end 68.834 34.9846) (width 0.254) (layer B.Cu) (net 1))
 (segment (start 66.2198 27.6925) (end 66.2198 32.3704) (width 0.254) (layer B.Cu) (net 1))
 (segment (start 65.5102 26.9829) (end 66.2198 27.6925) (width 0.254) (layer B.Cu) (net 1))
 (segment (start 61.0281 26.9829) (end 65.5102 26.9829) (width 0.254) (layer B.Cu) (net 1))
 (segment (start 59.944 28.067) (end 61.0281 26.9829) (width 0.254) (layer B.Cu) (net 1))
 (segment (start 68.834 36.0629) (end 68.834 34.9846) (width 0.254) (layer B.Cu) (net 1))
 (segment (start 65.3036 50.6108) (end 71.374 50.6108) (width 0.254) (layer B.Cu) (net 9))
 (segment (start 63.9834 49.2906) (end 65.3036 50.6108) (width 0.254) (layer B.Cu) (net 9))
 (segment (start 63.9834 45.9162) (end 63.9834 49.2906) (width 0.254) (layer B.Cu) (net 9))
 (segment (start 54.864 36.7968) (end 63.9834 45.9162) (width 0.254) (layer B.Cu) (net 9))
 (segment (start 54.864 28.067) (end 54.864 36.7968) (width 0.254) (layer B.Cu) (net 9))
 (segment (start 71.374 49.5325) (end 71.374 50.6108) (width 0.254) (layer B.Cu) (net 9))
 (segment (start 76.454 36.0629) (end 76.454 34.9846) (width 0.254) (layer B.Cu) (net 3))
 (segment (start 67.9439 26.4745) (end 76.454 34.9846) (width 0.254) (layer B.Cu) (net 3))
 (segment (start 58.9965 26.4745) (end 67.9439 26.4745) (width 0.254) (layer B.Cu) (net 3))
 (segment (start 57.404 28.067) (end 58.9965 26.4745) (width 0.254) (layer B.Cu) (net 3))
 (segment (start 79.8234 36.0673) (end 79.8234 38.354) (width 0.254) (layer B.Cu) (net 4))
 (segment (start 69.7136 25.9575) (end 79.8234 36.0673) (width 0.254) (layer B.Cu) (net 4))
 (segment (start 57.9031 25.9575) (end 69.7136 25.9575) (width 0.254) (layer B.Cu) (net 4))
 (segment (start 56.3189 27.5417) (end 57.9031 25.9575) (width 0.254) (layer B.Cu) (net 4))
 (segment (start 56.3189 28.5735) (end 56.3189 27.5417) (width 0.254) (layer B.Cu) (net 4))
 (segment (start 56.9052 29.1598) (end 56.3189 28.5735) (width 0.254) (layer B.Cu) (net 4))
 (segment (start 61.3912 29.1598) (end 56.9052 29.1598) (width 0.254) (layer B.Cu) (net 4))
 (segment (start 62.484 28.067) (end 61.3912 29.1598) (width 0.254) (layer B.Cu) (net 4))
 (segment (start 78.7451 38.354) (end 79.8234 38.354) (width 0.254) (layer B.Cu) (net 4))
 (segment (start 44.323 25.4) (end 44.323 28.472) (width 0.508) (layer B.Cu) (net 2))
 (segment (start 44.323 28.472) (end 44.2604 28.5346) (width 0.508) (layer B.Cu) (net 2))
 (via (at 71.6915 33.9051) (size 0.889) (layers F.Cu B.Cu) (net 2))
 (segment (start 44.2604 29.5096) (end 44.2604 29.1846) (width 0.508) (layer B.Cu) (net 2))
 (segment (start 32.766 35.179) (end 34.5836 35.179) (width 0.508) (layer B.Cu) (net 2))
 (segment (start 44.2604 29.5096) (end 36.6826 37.0874) (width 0.508) (layer B.Cu) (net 2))
 (segment (start 34.7742 35.179) (end 36.6826 37.0874) (width 0.508) (layer B.Cu) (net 2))
 (segment (start 34.5836 35.179) (end 34.7742 35.179) (width 0.508) (layer B.Cu) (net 2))
 (segment (start 38.735 39.1398) (end 38.735 52.07) (width 0.508) (layer B.Cu) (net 2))
 (segment (start 36.6826 37.0874) (end 38.735 39.1398) (width 0.508) (layer B.Cu) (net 2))
 (segment (start 44.2604 29.1846) (end 44.2604 28.5346) (width 0.508) (layer B.Cu) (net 2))
 (segment (start 44.2604 29.8346) (end 44.2604 29.5096) (width 0.508) (layer B.Cu) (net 2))
 (segment (start 72.644 36.0629) (end 72.644 34.8576) (width 0.508) (layer B.Cu) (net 2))
 (segment (start 32.766 35.179) (end 34.7742 35.179) (width 0.508) (layer F.Cu) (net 2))
 (segment (start 71.6915 33.9051) (end 72.644 34.8576) (width 0.508) (layer B.Cu) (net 2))
 (segment (start 36.0481 33.9051) (end 71.6915 33.9051) (width 0.508) (layer F.Cu) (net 2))
 (segment (start 34.7742 35.179) (end 36.0481 33.9051) (width 0.508) (layer F.Cu) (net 2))
 (segment (start 61.087 35.814) (end 48.387 35.814) (width 0.508) (layer F.Cu) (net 8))
 (segment (start 41.9097 40.259) (end 32.766 40.259) (width 0.508) (layer F.Cu) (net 8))
 (segment (start 46.3547 35.814) (end 41.9097 40.259) (width 0.508) (layer F.Cu) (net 8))
 (segment (start 48.387 35.814) (end 46.3547 35.814) (width 0.508) (layer F.Cu) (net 8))
 (segment (start 72.1214 51.2604) (end 72.644 50.7378) (width 0.508) (layer B.Cu) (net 8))
 (segment (start 63.7623 51.2604) (end 72.1214 51.2604) (width 0.508) (layer B.Cu) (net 8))
 (segment (start 50.4193 37.9174) (end 63.7623 51.2604) (width 0.508) (layer B.Cu) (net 8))
 (segment (start 50.4193 35.814) (end 50.4193 37.9174) (width 0.508) (layer B.Cu) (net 8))
 (segment (start 48.387 35.814) (end 50.4193 35.814) (width 0.508) (layer B.Cu) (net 8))
 (segment (start 72.644 49.5325) (end 72.644 50.7378) (width 0.508) (layer B.Cu) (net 8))
 (segment (start 65.024 33.9093) (end 63.1193 35.814) (width 0.508) (layer B.Cu) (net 8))
 (segment (start 65.024 28.067) (end 65.024 33.9093) (width 0.508) (layer B.Cu) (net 8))
 (segment (start 61.087 35.814) (end 63.1193 35.814) (width 0.508) (layer B.Cu) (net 8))
 (segment (start 66.2357 26.8553) (end 65.024 28.067) (width 0.508) (layer F.Cu) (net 8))
 (segment (start 80.857 26.8553) (end 66.2357 26.8553) (width 0.508) (layer F.Cu) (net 8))
 (segment (start 81.1747 27.173) (end 80.857 26.8553) (width 0.508) (layer F.Cu) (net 8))
 (segment (start 83.55 28.5444) (end 81.1747 27.173) (width 0.508) (layer F.Cu) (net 8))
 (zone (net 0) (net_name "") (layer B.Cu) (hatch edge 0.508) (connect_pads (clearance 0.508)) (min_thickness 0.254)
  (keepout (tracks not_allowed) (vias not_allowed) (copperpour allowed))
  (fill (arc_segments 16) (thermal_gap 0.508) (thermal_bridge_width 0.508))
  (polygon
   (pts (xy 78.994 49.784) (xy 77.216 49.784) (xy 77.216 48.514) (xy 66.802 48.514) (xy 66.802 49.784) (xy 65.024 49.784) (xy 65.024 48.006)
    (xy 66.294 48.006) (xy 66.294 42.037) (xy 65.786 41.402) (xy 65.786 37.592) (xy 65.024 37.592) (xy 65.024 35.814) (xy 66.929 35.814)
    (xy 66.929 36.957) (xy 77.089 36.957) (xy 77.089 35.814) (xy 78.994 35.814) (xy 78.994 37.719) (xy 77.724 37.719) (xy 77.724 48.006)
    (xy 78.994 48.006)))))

